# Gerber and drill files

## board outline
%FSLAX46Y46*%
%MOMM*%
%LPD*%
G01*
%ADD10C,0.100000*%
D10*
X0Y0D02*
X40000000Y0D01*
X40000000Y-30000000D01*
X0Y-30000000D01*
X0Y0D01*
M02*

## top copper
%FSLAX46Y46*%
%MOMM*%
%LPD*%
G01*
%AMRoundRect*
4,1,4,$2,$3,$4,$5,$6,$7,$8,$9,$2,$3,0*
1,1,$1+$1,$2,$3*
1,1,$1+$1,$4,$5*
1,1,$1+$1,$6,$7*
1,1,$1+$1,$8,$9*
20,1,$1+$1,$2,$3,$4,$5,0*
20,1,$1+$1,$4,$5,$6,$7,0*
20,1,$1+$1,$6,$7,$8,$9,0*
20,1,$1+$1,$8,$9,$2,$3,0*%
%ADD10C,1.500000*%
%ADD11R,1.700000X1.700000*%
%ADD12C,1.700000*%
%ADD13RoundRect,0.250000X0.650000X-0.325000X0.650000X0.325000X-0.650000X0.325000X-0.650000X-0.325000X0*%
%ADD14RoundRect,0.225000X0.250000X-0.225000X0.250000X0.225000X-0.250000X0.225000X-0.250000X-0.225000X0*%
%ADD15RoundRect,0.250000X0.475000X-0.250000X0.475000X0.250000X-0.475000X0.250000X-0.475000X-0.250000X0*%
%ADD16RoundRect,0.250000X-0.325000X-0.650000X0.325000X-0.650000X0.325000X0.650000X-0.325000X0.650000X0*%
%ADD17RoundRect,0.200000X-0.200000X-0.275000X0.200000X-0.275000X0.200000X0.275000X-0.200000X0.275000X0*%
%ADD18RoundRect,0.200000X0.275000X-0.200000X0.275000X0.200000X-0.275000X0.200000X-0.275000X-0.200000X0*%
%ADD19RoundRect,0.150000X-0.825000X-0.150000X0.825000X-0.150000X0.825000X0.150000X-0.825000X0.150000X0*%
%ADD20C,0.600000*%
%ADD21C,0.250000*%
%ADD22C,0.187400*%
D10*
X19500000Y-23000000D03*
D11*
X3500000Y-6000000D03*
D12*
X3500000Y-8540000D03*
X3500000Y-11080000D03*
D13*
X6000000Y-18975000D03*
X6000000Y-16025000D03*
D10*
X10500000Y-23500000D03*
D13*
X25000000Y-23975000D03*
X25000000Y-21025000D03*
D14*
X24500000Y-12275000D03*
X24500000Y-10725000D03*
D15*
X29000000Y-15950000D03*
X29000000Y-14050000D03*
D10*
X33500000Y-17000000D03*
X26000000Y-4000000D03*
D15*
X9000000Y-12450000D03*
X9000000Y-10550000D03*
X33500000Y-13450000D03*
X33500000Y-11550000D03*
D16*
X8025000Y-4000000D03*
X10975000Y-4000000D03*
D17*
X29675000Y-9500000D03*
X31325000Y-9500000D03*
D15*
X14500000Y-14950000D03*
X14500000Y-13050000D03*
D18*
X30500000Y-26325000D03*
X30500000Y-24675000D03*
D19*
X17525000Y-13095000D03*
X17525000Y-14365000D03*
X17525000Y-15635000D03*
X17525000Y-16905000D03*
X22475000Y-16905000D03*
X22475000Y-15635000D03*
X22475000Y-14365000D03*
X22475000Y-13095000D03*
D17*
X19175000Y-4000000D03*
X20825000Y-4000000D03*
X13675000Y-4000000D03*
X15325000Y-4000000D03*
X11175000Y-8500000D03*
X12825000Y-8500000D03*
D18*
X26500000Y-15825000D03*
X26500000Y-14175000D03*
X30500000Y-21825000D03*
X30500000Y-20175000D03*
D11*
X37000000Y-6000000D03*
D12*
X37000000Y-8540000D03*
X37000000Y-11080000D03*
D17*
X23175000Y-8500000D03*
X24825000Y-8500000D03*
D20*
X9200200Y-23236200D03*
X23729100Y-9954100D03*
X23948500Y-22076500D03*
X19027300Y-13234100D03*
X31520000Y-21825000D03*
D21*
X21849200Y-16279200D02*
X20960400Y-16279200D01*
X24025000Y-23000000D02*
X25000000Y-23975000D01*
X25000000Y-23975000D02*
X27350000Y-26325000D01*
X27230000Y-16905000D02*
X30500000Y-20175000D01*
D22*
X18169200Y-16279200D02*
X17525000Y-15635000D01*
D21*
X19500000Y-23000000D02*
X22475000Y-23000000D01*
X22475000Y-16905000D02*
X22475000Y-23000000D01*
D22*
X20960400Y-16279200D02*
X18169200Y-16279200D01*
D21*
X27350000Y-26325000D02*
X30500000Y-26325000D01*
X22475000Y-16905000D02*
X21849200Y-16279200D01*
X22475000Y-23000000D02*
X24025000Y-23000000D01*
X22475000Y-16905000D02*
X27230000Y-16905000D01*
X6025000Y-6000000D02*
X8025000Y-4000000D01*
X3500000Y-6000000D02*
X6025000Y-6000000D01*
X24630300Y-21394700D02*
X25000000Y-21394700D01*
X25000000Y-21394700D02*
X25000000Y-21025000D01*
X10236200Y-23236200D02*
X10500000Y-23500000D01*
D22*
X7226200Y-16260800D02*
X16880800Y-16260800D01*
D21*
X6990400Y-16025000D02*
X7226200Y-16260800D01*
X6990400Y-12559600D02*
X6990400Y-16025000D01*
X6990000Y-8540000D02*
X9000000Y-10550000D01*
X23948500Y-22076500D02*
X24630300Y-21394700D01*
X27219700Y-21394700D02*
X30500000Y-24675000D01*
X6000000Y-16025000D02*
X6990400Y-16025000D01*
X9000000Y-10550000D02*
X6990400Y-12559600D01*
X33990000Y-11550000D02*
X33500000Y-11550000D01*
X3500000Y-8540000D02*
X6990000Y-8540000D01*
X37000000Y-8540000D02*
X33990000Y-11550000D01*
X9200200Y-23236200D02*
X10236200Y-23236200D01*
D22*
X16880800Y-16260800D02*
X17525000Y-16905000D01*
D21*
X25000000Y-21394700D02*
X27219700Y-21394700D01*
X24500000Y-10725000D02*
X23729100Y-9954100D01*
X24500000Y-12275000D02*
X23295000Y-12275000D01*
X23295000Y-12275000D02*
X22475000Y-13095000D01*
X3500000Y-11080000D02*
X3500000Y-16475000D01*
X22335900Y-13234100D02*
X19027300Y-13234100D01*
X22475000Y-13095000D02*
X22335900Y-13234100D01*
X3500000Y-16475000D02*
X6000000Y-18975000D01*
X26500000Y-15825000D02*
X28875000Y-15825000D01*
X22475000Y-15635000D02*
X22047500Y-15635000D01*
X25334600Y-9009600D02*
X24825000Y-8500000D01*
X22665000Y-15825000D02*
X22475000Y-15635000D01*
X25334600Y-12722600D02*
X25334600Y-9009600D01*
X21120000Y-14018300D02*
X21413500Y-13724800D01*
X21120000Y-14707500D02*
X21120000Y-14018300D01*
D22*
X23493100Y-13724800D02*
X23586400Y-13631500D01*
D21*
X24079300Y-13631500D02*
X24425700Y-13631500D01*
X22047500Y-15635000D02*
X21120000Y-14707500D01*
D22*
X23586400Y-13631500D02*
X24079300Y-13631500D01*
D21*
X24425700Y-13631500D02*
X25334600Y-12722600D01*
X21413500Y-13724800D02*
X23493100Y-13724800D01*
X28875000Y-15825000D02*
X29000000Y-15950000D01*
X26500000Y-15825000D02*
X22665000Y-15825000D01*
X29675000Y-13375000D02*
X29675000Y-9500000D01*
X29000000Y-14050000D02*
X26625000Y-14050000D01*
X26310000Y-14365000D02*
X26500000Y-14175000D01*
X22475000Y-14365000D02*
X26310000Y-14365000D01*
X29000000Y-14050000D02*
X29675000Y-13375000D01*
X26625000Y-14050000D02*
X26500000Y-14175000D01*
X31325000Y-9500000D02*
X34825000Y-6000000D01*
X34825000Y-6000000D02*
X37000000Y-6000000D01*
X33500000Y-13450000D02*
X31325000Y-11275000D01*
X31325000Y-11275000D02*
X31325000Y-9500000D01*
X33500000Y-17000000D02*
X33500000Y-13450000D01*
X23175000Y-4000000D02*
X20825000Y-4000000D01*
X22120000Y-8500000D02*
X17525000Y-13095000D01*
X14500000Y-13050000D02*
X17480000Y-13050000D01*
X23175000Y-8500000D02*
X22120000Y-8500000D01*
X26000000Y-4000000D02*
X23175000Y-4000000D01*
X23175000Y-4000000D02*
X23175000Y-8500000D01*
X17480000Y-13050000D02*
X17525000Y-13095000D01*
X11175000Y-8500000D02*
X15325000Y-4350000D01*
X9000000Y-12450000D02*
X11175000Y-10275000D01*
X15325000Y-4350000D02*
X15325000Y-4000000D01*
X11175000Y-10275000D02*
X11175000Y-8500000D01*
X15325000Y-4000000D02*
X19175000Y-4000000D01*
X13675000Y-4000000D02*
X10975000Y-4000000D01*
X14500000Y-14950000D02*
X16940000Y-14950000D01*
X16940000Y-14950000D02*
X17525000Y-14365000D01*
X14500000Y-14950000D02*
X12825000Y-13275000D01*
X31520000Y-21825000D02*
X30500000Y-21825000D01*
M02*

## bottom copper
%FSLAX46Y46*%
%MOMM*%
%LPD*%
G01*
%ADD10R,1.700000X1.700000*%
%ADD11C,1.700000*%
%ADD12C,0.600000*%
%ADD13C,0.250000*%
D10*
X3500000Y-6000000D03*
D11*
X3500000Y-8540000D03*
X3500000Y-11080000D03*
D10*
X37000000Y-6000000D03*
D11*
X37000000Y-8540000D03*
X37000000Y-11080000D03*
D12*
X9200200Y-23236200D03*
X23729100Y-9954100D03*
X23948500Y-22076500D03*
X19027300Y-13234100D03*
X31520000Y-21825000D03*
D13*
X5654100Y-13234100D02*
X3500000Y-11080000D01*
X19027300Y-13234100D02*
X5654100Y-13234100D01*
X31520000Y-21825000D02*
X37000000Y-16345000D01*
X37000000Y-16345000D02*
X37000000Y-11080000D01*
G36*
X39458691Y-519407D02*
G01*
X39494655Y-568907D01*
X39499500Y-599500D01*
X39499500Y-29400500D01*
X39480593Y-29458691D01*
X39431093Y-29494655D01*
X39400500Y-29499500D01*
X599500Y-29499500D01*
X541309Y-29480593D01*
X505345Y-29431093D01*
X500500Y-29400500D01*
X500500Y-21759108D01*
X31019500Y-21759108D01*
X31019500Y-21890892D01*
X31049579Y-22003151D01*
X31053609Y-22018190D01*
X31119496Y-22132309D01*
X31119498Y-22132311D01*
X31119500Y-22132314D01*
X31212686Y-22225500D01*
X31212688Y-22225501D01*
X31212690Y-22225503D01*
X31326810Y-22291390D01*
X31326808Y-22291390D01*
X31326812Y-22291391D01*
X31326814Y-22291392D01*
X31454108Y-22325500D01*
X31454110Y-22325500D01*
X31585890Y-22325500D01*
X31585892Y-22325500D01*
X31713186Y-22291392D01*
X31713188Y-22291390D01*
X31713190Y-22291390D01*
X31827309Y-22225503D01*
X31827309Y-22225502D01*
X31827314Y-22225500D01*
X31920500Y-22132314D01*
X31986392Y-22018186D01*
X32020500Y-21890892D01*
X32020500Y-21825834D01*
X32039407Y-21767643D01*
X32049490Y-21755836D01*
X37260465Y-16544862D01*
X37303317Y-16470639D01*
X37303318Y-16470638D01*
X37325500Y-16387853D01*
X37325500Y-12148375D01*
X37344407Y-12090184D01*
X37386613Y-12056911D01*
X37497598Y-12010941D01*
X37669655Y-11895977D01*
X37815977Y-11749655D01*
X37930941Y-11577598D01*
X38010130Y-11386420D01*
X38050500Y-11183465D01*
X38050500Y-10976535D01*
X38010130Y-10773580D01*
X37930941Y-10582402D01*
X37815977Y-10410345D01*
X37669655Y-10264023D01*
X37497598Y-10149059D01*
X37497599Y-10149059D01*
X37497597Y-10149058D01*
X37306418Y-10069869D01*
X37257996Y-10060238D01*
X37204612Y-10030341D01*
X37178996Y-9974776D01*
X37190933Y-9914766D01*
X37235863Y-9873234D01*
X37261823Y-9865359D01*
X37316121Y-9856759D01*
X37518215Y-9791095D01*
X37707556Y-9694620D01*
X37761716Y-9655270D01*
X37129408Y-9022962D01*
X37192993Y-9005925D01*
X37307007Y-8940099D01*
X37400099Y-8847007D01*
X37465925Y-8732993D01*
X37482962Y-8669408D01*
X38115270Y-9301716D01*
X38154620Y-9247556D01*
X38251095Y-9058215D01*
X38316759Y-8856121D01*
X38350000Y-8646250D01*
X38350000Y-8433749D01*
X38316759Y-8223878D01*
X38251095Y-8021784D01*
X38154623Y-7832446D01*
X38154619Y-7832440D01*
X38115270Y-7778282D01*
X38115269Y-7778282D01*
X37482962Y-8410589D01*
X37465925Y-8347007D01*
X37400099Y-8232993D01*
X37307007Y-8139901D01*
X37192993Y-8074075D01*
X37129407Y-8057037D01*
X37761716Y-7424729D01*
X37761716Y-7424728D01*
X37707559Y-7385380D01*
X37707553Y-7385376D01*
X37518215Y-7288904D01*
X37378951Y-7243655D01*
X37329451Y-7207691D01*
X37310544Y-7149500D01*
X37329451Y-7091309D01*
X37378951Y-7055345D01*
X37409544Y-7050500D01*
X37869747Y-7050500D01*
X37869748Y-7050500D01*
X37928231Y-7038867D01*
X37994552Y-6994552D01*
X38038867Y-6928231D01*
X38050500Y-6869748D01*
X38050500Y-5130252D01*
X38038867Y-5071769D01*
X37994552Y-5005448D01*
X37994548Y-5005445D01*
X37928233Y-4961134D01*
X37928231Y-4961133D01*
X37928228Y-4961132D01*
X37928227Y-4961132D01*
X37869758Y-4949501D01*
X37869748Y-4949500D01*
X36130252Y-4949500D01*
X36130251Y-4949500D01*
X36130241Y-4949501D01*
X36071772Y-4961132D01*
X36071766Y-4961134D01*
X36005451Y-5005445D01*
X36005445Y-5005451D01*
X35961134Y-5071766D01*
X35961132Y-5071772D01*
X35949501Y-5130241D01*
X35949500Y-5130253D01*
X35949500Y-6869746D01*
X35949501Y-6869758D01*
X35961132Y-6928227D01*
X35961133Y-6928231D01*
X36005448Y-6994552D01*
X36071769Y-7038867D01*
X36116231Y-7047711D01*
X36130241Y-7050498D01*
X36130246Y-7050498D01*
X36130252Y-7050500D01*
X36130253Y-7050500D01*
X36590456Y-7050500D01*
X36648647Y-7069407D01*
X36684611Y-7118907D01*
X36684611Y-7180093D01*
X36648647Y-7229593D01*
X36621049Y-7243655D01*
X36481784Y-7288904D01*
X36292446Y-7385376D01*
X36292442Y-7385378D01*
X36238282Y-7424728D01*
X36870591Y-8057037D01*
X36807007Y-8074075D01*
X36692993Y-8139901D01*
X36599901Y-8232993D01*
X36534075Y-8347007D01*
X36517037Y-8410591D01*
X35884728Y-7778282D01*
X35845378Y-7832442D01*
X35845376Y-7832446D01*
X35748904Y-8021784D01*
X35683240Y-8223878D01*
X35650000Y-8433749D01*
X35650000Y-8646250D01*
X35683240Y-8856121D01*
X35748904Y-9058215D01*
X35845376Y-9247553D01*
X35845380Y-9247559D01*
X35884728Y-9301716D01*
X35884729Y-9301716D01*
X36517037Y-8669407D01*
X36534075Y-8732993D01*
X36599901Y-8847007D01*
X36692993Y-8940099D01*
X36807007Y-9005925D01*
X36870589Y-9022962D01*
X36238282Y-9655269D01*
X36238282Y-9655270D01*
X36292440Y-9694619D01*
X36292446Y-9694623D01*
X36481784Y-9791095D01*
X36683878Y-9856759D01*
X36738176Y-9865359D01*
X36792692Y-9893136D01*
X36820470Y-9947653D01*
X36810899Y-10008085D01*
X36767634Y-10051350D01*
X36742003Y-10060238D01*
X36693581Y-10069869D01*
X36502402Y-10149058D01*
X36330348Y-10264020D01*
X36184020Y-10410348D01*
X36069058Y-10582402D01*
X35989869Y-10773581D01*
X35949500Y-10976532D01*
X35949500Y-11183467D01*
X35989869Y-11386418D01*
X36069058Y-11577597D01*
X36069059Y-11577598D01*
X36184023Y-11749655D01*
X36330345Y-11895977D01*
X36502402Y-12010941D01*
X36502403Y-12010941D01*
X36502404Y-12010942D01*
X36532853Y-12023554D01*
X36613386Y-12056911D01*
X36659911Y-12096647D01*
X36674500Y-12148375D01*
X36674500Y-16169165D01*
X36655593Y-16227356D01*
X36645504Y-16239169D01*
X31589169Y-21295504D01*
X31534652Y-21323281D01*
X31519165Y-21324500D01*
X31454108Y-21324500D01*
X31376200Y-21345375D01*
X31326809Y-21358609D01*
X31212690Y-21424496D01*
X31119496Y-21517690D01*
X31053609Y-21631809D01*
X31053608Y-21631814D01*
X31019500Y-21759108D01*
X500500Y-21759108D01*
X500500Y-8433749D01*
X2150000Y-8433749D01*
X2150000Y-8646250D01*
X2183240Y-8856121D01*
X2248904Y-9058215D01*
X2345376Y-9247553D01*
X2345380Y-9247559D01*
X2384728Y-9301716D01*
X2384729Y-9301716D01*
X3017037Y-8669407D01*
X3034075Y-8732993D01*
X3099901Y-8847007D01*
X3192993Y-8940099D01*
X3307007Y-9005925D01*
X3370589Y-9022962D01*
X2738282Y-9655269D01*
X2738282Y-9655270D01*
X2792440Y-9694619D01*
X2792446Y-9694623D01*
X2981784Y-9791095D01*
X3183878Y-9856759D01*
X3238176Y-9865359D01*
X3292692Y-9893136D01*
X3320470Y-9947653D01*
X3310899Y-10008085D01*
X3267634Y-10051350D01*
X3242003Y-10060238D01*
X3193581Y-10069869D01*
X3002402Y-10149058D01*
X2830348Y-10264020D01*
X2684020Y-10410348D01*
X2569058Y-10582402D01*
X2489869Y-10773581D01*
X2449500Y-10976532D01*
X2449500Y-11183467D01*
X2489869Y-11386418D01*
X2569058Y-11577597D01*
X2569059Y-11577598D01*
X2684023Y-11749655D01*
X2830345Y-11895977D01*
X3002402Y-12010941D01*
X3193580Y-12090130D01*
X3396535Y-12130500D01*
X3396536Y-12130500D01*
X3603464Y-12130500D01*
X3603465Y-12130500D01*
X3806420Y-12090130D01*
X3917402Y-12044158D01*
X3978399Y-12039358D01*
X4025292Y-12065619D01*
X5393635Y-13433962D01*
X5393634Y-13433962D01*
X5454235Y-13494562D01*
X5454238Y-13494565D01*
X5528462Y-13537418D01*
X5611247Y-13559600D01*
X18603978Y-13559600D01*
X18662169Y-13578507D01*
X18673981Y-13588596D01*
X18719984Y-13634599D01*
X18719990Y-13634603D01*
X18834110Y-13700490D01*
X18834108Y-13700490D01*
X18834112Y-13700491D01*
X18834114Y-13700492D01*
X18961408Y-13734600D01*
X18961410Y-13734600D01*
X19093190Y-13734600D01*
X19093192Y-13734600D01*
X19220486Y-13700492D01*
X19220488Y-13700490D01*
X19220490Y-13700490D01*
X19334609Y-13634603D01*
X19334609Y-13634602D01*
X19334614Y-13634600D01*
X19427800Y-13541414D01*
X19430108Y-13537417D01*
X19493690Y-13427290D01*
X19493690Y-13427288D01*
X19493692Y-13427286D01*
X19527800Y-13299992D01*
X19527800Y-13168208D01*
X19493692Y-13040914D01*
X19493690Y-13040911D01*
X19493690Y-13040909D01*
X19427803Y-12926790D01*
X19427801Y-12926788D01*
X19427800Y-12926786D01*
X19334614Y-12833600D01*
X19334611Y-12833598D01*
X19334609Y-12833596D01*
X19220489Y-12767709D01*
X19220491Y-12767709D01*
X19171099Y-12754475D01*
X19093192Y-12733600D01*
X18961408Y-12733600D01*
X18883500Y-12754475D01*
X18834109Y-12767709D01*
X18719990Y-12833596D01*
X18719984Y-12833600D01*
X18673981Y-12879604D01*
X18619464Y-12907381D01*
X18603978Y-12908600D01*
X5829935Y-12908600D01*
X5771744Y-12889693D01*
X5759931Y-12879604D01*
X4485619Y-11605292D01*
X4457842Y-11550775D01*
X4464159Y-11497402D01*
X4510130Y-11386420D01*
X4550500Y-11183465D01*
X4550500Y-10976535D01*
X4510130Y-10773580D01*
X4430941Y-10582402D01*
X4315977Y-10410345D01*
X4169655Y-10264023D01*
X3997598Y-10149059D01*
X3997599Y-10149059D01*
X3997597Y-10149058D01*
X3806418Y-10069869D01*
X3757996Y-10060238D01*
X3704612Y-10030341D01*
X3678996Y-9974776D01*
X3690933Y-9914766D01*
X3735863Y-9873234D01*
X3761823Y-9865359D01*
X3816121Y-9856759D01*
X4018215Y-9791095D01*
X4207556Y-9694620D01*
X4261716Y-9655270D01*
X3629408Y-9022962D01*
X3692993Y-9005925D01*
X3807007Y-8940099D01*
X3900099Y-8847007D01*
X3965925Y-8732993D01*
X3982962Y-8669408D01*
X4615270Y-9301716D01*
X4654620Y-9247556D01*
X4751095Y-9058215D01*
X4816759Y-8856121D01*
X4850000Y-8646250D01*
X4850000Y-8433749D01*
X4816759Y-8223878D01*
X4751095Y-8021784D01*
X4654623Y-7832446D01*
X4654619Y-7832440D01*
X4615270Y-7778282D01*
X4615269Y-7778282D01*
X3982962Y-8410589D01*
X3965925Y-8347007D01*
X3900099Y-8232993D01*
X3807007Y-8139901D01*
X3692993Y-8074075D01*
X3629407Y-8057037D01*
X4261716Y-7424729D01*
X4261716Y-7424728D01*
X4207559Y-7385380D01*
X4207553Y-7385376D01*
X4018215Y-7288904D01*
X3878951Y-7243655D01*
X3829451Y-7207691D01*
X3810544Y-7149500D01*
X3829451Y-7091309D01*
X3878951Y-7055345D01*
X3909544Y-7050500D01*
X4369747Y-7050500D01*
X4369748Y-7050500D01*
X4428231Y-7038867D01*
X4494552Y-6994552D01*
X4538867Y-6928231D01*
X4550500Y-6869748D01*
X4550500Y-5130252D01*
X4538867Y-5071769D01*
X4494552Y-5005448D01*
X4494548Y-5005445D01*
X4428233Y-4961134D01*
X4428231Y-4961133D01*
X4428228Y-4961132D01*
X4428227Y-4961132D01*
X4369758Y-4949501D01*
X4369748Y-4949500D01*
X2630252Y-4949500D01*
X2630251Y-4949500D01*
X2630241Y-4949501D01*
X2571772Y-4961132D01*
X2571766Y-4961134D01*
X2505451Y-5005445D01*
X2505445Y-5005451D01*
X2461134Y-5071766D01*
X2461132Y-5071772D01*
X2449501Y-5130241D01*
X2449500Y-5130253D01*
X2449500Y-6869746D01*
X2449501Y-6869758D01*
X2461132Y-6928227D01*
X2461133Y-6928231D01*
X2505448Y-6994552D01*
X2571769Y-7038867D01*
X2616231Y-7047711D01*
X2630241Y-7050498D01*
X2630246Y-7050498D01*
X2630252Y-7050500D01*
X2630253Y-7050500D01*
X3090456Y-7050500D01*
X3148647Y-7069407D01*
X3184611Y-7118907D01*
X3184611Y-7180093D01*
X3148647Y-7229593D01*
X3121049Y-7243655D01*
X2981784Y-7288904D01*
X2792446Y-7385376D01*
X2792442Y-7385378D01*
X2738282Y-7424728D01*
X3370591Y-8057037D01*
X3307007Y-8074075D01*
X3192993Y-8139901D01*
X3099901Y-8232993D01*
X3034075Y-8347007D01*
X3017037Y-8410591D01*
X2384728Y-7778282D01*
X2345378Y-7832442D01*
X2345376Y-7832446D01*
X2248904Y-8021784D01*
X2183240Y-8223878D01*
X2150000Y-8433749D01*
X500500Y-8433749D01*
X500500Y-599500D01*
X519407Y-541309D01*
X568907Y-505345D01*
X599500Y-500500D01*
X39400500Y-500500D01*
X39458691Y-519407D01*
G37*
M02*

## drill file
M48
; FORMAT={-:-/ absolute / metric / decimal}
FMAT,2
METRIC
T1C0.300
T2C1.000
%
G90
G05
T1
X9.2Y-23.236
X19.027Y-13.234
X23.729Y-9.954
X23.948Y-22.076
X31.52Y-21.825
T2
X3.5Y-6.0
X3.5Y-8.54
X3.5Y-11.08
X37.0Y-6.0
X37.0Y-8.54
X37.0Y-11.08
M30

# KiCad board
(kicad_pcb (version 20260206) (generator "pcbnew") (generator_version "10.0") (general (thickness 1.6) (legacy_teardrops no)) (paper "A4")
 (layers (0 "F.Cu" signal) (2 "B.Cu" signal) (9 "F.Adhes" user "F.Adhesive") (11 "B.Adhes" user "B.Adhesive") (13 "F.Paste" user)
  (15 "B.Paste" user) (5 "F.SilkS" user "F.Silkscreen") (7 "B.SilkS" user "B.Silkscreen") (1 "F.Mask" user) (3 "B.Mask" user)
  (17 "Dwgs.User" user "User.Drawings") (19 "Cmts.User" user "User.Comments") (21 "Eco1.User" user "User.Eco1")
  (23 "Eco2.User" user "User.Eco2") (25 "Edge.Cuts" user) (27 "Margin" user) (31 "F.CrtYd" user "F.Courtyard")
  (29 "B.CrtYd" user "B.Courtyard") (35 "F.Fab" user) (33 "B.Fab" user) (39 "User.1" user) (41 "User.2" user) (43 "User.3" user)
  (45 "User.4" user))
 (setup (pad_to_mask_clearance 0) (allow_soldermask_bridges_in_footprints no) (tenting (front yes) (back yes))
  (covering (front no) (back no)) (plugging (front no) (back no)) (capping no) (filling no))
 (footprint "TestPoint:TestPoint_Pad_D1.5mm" (layer "F.Cu") (at 19.5 23)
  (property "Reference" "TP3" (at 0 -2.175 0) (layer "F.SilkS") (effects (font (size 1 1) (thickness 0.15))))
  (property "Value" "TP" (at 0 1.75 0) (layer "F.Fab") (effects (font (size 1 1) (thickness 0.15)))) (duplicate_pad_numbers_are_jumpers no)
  (pad "1" smd circle (at 0 0) (size 1.5 1.5) (layers "F.Cu" "F.Mask") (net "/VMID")))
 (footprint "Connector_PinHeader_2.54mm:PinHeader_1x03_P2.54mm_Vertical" (layer "F.Cu") (at 3.5 6)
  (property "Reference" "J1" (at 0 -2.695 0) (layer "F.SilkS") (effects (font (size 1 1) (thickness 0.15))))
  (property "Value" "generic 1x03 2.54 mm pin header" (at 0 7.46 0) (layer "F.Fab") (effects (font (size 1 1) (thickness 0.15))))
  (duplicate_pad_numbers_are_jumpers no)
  (pad "1" thru_hole rect (at 0 0) (size 1.7 1.7) (drill 1) (layers "*.Cu" "*.Mask") (remove_unused_layers no) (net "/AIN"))
  (pad "2" thru_hole circle (at 0 2.54) (size 1.7 1.7) (drill 1) (layers "*.Cu" "*.Mask") (remove_unused_layers no) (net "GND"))
  (pad "3" thru_hole circle (at 0 5.08) (size 1.7 1.7) (drill 1) (layers "*.Cu" "*.Mask") (remove_unused_layers no) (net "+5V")))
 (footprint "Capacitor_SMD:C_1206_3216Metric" (layer "F.Cu") (at 6 17.5 90)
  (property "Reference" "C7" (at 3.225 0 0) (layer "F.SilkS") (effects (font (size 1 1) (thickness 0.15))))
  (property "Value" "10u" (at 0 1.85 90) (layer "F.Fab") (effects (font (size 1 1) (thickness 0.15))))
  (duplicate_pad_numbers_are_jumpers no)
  (pad "1" smd roundrect (at -1.475 0 90) (size 1.15 1.8) (layers "F.Cu" "F.Mask" "F.Paste") (roundrect_rratio 0.217391) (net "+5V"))
  (pad "2" smd roundrect (at 1.475 0 90) (size 1.15 1.8) (layers "F.Cu" "F.Mask" "F.Paste") (roundrect_rratio 0.217391) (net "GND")))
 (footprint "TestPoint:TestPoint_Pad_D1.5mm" (layer "F.Cu") (at 10.5 23.5)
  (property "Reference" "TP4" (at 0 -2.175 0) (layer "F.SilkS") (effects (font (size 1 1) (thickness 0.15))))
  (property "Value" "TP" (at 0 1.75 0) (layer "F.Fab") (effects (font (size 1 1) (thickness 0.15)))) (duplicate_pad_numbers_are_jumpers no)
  (pad "1" smd circle (at 0 0) (size 1.5 1.5) (layers "F.Cu" "F.Mask") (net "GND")))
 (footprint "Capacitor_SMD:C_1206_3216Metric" (layer "F.Cu") (at 25 22.5 90)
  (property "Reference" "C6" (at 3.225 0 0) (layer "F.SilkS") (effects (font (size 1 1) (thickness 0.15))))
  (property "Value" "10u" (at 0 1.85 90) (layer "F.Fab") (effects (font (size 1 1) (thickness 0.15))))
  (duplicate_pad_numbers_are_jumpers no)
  (pad "1" smd roundrect (at -1.475 0 90) (size 1.15 1.8) (layers "F.Cu" "F.Mask" "F.Paste") (roundrect_rratio 0.217391) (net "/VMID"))
  (pad "2" smd roundrect (at 1.475 0 90) (size 1.15 1.8) (layers "F.Cu" "F.Mask" "F.Paste") (roundrect_rratio 0.217391) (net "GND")))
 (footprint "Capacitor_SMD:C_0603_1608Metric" (layer "F.Cu") (at 24.5 11.5 90)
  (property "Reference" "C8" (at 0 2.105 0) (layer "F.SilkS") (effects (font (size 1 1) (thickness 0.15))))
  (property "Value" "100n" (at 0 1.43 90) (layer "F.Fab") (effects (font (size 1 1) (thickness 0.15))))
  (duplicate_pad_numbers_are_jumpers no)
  (pad "1" smd roundrect (at -0.775 0 90) (size 0.9 0.95) (layers "F.Cu" "F.Mask" "F.Paste") (roundrect_rratio 0.25) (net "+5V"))
  (pad "2" smd roundrect (at 0.775 0 90) (size 0.9 0.95) (layers "F.Cu" "F.Mask" "F.Paste") (roundrect_rratio 0.25) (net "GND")))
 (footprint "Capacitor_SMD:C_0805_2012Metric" (layer "F.Cu") (at 29 15 90)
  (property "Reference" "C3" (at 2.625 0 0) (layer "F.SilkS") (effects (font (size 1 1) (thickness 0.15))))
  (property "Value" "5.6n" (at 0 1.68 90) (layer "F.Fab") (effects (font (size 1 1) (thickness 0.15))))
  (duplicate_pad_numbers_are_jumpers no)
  (pad "1" smd roundrect (at -0.95 0 90) (size 1 1.45) (layers "F.Cu" "F.Mask" "F.Paste") (roundrect_rratio 0.25) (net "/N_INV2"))
  (pad "2" smd roundrect (at 0.95 0 90) (size 1 1.45) (layers "F.Cu" "F.Mask" "F.Paste") (roundrect_rratio 0.25) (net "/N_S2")))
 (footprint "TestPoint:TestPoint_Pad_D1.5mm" (layer "F.Cu") (at 33.5 17)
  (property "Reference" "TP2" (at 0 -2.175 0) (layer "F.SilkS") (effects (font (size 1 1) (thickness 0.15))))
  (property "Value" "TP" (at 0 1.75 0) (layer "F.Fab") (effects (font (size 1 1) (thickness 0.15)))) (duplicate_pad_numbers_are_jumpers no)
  (pad "1" smd circle (at 0 0) (size 1.5 1.5) (layers "F.Cu" "F.Mask") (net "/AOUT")))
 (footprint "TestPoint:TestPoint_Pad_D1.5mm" (layer "F.Cu") (at 26 4)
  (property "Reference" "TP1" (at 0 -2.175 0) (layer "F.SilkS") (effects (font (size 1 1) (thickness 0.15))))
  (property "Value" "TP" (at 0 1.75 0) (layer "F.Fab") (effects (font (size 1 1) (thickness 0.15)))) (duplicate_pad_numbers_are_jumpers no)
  (pad "1" smd circle (at 0 0) (size 1.5 1.5) (layers "F.Cu" "F.Mask") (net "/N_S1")))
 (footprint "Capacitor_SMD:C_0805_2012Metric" (layer "F.Cu") (at 9 11.5 90)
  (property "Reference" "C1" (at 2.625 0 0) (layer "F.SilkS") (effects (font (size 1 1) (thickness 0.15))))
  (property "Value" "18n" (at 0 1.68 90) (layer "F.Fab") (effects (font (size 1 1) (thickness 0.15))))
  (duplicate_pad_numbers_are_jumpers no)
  (pad "1" smd roundrect (at -0.95 0 90) (size 1 1.45) (layers "F.Cu" "F.Mask" "F.Paste") (roundrect_rratio 0.25) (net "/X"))
  (pad "2" smd roundrect (at 0.95 0 90) (size 1 1.45) (layers "F.Cu" "F.Mask" "F.Paste") (roundrect_rratio 0.25) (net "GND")))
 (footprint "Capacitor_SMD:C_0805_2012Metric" (layer "F.Cu") (at 33.5 12.5 90)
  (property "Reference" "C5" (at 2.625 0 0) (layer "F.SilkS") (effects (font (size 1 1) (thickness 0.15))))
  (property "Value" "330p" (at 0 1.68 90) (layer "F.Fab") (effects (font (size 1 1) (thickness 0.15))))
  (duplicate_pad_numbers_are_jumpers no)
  (pad "1" smd roundrect (at -0.95 0 90) (size 1 1.45) (layers "F.Cu" "F.Mask" "F.Paste") (roundrect_rratio 0.25) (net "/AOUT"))
  (pad "2" smd roundrect (at 0.95 0 90) (size 1 1.45) (layers "F.Cu" "F.Mask" "F.Paste") (roundrect_rratio 0.25) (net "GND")))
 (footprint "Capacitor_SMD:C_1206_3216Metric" (layer "F.Cu") (at 9.5 4)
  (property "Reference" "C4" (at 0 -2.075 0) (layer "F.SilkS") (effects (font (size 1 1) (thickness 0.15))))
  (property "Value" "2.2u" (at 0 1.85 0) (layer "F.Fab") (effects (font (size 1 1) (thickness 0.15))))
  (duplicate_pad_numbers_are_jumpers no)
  (pad "1" smd roundrect (at -1.475 0) (size 1.15 1.8) (layers "F.Cu" "F.Mask" "F.Paste") (roundrect_rratio 0.217391) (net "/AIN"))
  (pad "2" smd roundrect (at 1.475 0) (size 1.15 1.8) (layers "F.Cu" "F.Mask" "F.Paste") (roundrect_rratio 0.217391) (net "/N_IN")))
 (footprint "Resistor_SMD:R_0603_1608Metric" (layer "F.Cu") (at 30.5 9.5)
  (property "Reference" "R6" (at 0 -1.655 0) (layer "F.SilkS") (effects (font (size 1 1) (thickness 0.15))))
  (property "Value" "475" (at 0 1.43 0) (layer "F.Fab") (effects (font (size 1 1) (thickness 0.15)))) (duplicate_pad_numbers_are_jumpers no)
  (pad "1" smd roundrect (at -0.825 0) (size 0.8 0.95) (layers "F.Cu" "F.Mask" "F.Paste") (roundrect_rratio 0.25) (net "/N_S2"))
  (pad "2" smd roundrect (at 0.825 0) (size 0.8 0.95) (layers "F.Cu" "F.Mask" "F.Paste") (roundrect_rratio 0.25) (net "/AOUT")))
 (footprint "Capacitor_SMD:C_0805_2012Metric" (layer "F.Cu") (at 14.5 14 90)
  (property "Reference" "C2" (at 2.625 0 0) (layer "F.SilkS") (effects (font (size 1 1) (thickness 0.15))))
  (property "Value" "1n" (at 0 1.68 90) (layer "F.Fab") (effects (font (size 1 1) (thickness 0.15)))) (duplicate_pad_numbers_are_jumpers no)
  (pad "1" smd roundrect (at -0.95 0 90) (size 1 1.45) (layers "F.Cu" "F.Mask" "F.Paste") (roundrect_rratio 0.25) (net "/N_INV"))
  (pad "2" smd roundrect (at 0.95 0 90) (size 1 1.45) (layers "F.Cu" "F.Mask" "F.Paste") (roundrect_rratio 0.25) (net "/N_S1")))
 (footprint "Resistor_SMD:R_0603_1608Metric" (layer "F.Cu") (at 30.5 25.5 90)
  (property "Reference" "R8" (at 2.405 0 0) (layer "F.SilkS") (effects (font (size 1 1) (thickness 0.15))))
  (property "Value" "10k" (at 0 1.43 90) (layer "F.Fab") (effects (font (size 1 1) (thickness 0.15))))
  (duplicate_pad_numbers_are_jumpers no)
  (pad "1" smd roundrect (at -0.825 0 90) (size 0.8 0.95) (layers "F.Cu" "F.Mask" "F.Paste") (roundrect_rratio 0.25) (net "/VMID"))
  (pad "2" smd roundrect (at 0.825 0 90) (size 0.8 0.95) (layers "F.Cu" "F.Mask" "F.Paste") (roundrect_rratio 0.25) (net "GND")))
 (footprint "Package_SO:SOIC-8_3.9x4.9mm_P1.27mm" (layer "F.Cu") (at 20 15)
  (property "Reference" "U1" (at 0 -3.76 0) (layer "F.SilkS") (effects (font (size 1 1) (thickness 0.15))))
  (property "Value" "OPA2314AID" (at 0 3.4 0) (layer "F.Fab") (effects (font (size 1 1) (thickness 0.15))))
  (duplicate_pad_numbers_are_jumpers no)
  (pad "1" smd roundrect (at -2.475 -1.905) (size 1.95 0.6) (layers "F.Cu" "F.Mask" "F.Paste") (roundrect_rratio 0.25) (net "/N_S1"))
  (pad "2" smd roundrect (at -2.475 -0.635) (size 1.95 0.6) (layers "F.Cu" "F.Mask" "F.Paste") (roundrect_rratio 0.25) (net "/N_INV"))
  (pad "3" smd roundrect (at -2.475 0.635) (size 1.95 0.6) (layers "F.Cu" "F.Mask" "F.Paste") (roundrect_rratio 0.25) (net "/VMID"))
  (pad "4" smd roundrect (at -2.475 1.905) (size 1.95 0.6) (layers "F.Cu" "F.Mask" "F.Paste") (roundrect_rratio 0.25) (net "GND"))
  (pad "5" smd roundrect (at 2.475 1.905) (size 1.95 0.6) (layers "F.Cu" "F.Mask" "F.Paste") (roundrect_rratio 0.25) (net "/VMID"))
  (pad "6" smd roundrect (at 2.475 0.635) (size 1.95 0.6) (layers "F.Cu" "F.Mask" "F.Paste") (roundrect_rratio 0.25) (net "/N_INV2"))
  (pad "7" smd roundrect (at 2.475 -0.635) (size 1.95 0.6) (layers "F.Cu" "F.Mask" "F.Paste") (roundrect_rratio 0.25) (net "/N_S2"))
  (pad "8" smd roundrect (at 2.475 -1.905) (size 1.95 0.6) (layers "F.Cu" "F.Mask" "F.Paste") (roundrect_rratio 0.25) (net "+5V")))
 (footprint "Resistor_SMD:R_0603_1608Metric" (layer "F.Cu") (at 20 4)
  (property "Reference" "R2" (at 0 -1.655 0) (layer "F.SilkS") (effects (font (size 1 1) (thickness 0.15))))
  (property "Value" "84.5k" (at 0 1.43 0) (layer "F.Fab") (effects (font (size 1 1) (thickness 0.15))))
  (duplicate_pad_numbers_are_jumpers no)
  (pad "1" smd roundrect (at -0.825 0) (size 0.8 0.95) (layers "F.Cu" "F.Mask" "F.Paste") (roundrect_rratio 0.25) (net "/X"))
  (pad "2" smd roundrect (at 0.825 0) (size 0.8 0.95) (layers "F.Cu" "F.Mask" "F.Paste") (roundrect_rratio 0.25) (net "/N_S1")))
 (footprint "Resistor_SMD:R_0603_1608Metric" (layer "F.Cu") (at 14.5 4)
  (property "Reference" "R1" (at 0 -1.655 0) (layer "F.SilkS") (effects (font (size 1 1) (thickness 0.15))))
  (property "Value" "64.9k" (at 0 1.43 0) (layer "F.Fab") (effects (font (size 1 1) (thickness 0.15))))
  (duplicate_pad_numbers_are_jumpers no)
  (pad "1" smd roundrect (at -0.825 0) (size 0.8 0.95) (layers "F.Cu" "F.Mask" "F.Paste") (roundrect_rratio 0.25) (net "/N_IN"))
  (pad "2" smd roundrect (at 0.825 0) (size 0.8 0.95) (layers "F.Cu" "F.Mask" "F.Paste") (roundrect_rratio 0.25) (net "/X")))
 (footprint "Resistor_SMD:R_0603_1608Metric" (layer "F.Cu") (at 12 8.5)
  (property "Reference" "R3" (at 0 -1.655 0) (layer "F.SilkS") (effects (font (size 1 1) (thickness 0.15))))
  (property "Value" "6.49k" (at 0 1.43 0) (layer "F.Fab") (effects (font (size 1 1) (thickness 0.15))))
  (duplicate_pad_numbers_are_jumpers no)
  (pad "1" smd roundrect (at -0.825 0) (size 0.8 0.95) (layers "F.Cu" "F.Mask" "F.Paste") (roundrect_rratio 0.25) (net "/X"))
  (pad "2" smd roundrect (at 0.825 0) (size 0.8 0.95) (layers "F.Cu" "F.Mask" "F.Paste") (roundrect_rratio 0.25) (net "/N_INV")))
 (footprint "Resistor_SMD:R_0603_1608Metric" (layer "F.Cu") (at 26.5 15 90)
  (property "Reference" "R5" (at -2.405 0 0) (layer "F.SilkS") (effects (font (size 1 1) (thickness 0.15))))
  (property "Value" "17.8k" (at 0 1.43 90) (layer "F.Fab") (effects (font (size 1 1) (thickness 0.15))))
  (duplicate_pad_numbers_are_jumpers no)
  (pad "1" smd roundrect (at -0.825 0 90) (size 0.8 0.95) (layers "F.Cu" "F.Mask" "F.Paste") (roundrect_rratio 0.25) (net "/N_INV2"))
  (pad "2" smd roundrect (at 0.825 0 90) (size 0.8 0.95) (layers "F.Cu" "F.Mask" "F.Paste") (roundrect_rratio 0.25) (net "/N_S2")))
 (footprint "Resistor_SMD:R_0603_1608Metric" (layer "F.Cu") (at 30.5 21 90)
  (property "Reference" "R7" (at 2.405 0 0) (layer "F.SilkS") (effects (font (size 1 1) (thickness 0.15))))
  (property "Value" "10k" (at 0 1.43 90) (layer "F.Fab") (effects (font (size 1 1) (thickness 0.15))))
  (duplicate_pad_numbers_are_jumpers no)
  (pad "1" smd roundrect (at -0.825 0 90) (size 0.8 0.95) (layers "F.Cu" "F.Mask" "F.Paste") (roundrect_rratio 0.25) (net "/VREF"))
  (pad "2" smd roundrect (at 0.825 0 90) (size 0.8 0.95) (layers "F.Cu" "F.Mask" "F.Paste") (roundrect_rratio 0.25) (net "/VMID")))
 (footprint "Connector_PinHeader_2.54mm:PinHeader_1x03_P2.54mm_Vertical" (layer "F.Cu") (at 37 6)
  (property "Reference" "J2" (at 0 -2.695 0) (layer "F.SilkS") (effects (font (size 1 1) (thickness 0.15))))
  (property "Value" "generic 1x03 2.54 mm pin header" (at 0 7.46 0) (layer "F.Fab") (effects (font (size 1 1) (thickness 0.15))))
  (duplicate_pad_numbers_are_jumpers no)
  (pad "1" thru_hole rect (at 0 0) (size 1.7 1.7) (drill 1) (layers "*.Cu" "*.Mask") (remove_unused_layers no) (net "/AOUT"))
  (pad "2" thru_hole circle (at 0 2.54) (size 1.7 1.7) (drill 1) (layers "*.Cu" "*.Mask") (remove_unused_layers no) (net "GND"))
  (pad "3" thru_hole circle (at 0 5.08) (size 1.7 1.7) (drill 1) (layers "*.Cu" "*.Mask") (remove_unused_layers no) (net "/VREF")))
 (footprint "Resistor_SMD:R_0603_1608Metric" (layer "F.Cu") (at 24 8.5)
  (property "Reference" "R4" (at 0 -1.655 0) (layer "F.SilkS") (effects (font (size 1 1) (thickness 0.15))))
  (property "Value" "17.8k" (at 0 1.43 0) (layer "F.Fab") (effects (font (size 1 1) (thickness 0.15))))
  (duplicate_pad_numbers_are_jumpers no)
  (pad "1" smd roundrect (at -0.825 0) (size 0.8 0.95) (layers "F.Cu" "F.Mask" "F.Paste") (roundrect_rratio 0.25) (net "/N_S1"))
  (pad "2" smd roundrect (at 0.825 0) (size 0.8 0.95) (layers "F.Cu" "F.Mask" "F.Paste") (roundrect_rratio 0.25) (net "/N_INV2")))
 (gr_rect (start 0 0) (end 40 30) (stroke (width 0.1) (type default)) (fill no) (layer "Edge.Cuts"))
 (segment (start 21.8492 16.2792) (end 20.9604 16.2792) (width 0.25) (layer "F.Cu") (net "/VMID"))
 (segment (start 24.025 23) (end 25 23.975) (width 0.25) (layer "F.Cu") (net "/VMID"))
 (segment (start 25 23.975) (end 27.35 26.325) (width 0.25) (layer "F.Cu") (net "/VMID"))
 (segment (start 27.23 16.905) (end 30.5 20.175) (width 0.25) (layer "F.Cu") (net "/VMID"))
 (segment (start 18.1692 16.2792) (end 17.525 15.635) (width 0.1874) (layer "F.Cu") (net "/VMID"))
 (segment (start 19.5 23) (end 22.475 23) (width 0.25) (layer "F.Cu") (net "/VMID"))
 (segment (start 22.475 16.905) (end 22.475 23) (width 0.25) (layer "F.Cu") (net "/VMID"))
 (segment (start 20.9604 16.2792) (end 18.1692 16.2792) (width 0.1874) (layer "F.Cu") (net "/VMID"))
 (segment (start 27.35 26.325) (end 30.5 26.325) (width 0.25) (layer "F.Cu") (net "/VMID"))
 (segment (start 22.475 16.905) (end 21.8492 16.2792) (width 0.25) (layer "F.Cu") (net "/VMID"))
 (segment (start 22.475 23) (end 24.025 23) (width 0.25) (layer "F.Cu") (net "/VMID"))
 (segment (start 22.475 16.905) (end 27.23 16.905) (width 0.25) (layer "F.Cu") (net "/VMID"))
 (segment (start 6.025 6) (end 8.025 4) (width 0.25) (layer "F.Cu") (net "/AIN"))
 (segment (start 3.5 6) (end 6.025 6) (width 0.25) (layer "F.Cu") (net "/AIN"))
 (segment (start 24.6303 21.3947) (end 25 21.3947) (width 0.25) (layer "F.Cu") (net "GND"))
 (segment (start 25 21.3947) (end 25 21.025) (width 0.25) (layer "F.Cu") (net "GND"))
 (segment (start 10.2362 23.2362) (end 10.5 23.5) (width 0.25) (layer "F.Cu") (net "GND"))
 (segment (start 7.2262 16.2608) (end 16.8808 16.2608) (width 0.1874) (layer "F.Cu") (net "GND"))
 (segment (start 6.9904 16.025) (end 7.2262 16.2608) (width 0.25) (layer "F.Cu") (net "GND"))
 (segment (start 6.9904 12.5596) (end 6.9904 16.025) (width 0.25) (layer "F.Cu") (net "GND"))
 (segment (start 6.99 8.54) (end 9 10.55) (width 0.25) (layer "F.Cu") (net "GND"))
 (segment (start 23.9485 22.0765) (end 24.6303 21.3947) (width 0.25) (layer "F.Cu") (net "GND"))
 (segment (start 27.2197 21.3947) (end 30.5 24.675) (width 0.25) (layer "F.Cu") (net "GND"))
 (segment (start 6 16.025) (end 6.9904 16.025) (width 0.25) (layer "F.Cu") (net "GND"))
 (segment (start 9 10.55) (end 6.9904 12.5596) (width 0.25) (layer "F.Cu") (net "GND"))
 (segment (start 33.99 11.55) (end 33.5 11.55) (width 0.25) (layer "F.Cu") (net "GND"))
 (segment (start 3.5 8.54) (end 6.99 8.54) (width 0.25) (layer "F.Cu") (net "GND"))
 (segment (start 37 8.54) (end 33.99 11.55) (width 0.25) (layer "F.Cu") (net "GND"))
 (segment (start 9.2002 23.2362) (end 10.2362 23.2362) (width 0.25) (layer "F.Cu") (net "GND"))
 (segment (start 16.8808 16.2608) (end 17.525 16.905) (width 0.1874) (layer "F.Cu") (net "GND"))
 (segment (start 25 21.3947) (end 27.2197 21.3947) (width 0.25) (layer "F.Cu") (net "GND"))
 (segment (start 24.5 10.725) (end 23.7291 9.9541) (width 0.25) (layer "F.Cu") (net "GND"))
 (via (at 9.2002 23.2362) (size 0.6) (drill 0.3) (layers "F.Cu" "B.Cu") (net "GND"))
 (via (at 23.7291 9.9541) (size 0.6) (drill 0.3) (layers "F.Cu" "B.Cu") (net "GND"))
 (via (at 23.9485 22.0765) (size 0.6) (drill 0.3) (layers "F.Cu" "B.Cu") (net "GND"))
 (segment (start 24.5 12.275) (end 23.295 12.275) (width 0.25) (layer "F.Cu") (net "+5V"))
 (segment (start 23.295 12.275) (end 22.475 13.095) (width 0.25) (layer "F.Cu") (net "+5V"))
 (segment (start 3.5 11.08) (end 3.5 16.475) (width 0.25) (layer "F.Cu") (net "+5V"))
 (segment (start 22.3359 13.2341) (end 19.0273 13.2341) (width 0.25) (layer "F.Cu") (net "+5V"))
 (segment (start 22.475 13.095) (end 22.3359 13.2341) (width 0.25) (layer "F.Cu") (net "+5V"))
 (segment (start 3.5 16.475) (end 6 18.975) (width 0.25) (layer "F.Cu") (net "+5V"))
 (via (at 19.0273 13.2341) (size 0.6) (drill 0.3) (layers "F.Cu" "B.Cu") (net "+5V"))
 (segment (start 5.6541 13.2341) (end 3.5 11.08) (width 0.25) (layer "B.Cu") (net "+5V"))
 (segment (start 19.0273 13.2341) (end 5.6541 13.2341) (width 0.25) (layer "B.Cu") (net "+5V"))
 (segment (start 26.5 15.825) (end 28.875 15.825) (width 0.25) (layer "F.Cu") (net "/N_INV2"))
 (segment (start 22.475 15.635) (end 22.0475 15.635) (width 0.25) (layer "F.Cu") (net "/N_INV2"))
 (segment (start 25.3346 9.0096) (end 24.825 8.5) (width 0.25) (layer "F.Cu") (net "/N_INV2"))
 (segment (start 22.665 15.825) (end 22.475 15.635) (width 0.25) (layer "F.Cu") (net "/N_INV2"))
 (segment (start 25.3346 12.7226) (end 25.3346 9.0096) (width 0.25) (layer "F.Cu") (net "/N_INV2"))
 (segment (start 21.12 14.0183) (end 21.4135 13.7248) (width 0.25) (layer "F.Cu") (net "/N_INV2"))
 (segment (start 21.12 14.7075) (end 21.12 14.0183) (width 0.25) (layer "F.Cu") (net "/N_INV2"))
 (segment (start 23.4931 13.7248) (end 23.5864 13.6315) (width 0.1874) (layer "F.Cu") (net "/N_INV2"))
 (segment (start 24.0793 13.6315) (end 24.4257 13.6315) (width 0.25) (layer "F.Cu") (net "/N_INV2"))
 (segment (start 22.0475 15.635) (end 21.12 14.7075) (width 0.25) (layer "F.Cu") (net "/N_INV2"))
 (segment (start 23.5864 13.6315) (end 24.0793 13.6315) (width 0.1874) (layer "F.Cu") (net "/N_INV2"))
 (segment (start 24.4257 13.6315) (end 25.3346 12.7226) (width 0.25) (layer "F.Cu") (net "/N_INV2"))
 (segment (start 21.4135 13.7248) (end 23.4931 13.7248) (width 0.25) (layer "F.Cu") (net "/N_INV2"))
 (segment (start 28.875 15.825) (end 29 15.95) (width 0.25) (layer "F.Cu") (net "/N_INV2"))
 (segment (start 26.5 15.825) (end 22.665 15.825) (width 0.25) (layer "F.Cu") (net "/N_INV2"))
 (segment (start 29.675 13.375) (end 29.675 9.5) (width 0.25) (layer "F.Cu") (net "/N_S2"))
 (segment (start 29 14.05) (end 26.625 14.05) (width 0.25) (layer "F.Cu") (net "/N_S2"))
 (segment (start 26.31 14.365) (end 26.5 14.175) (width 0.25) (layer "F.Cu") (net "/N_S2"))
 (segment (start 22.475 14.365) (end 26.31 14.365) (width 0.25) (layer "F.Cu") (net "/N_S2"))
 (segment (start 29 14.05) (end 29.675 13.375) (width 0.25) (layer "F.Cu") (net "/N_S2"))
 (segment (start 26.625 14.05) (end 26.5 14.175) (width 0.25) (layer "F.Cu") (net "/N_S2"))
 (segment (start 31.325 9.5) (end 34.825 6) (width 0.25) (layer "F.Cu") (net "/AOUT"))
 (segment (start 34.825 6) (end 37 6) (width 0.25) (layer "F.Cu") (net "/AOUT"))
 (segment (start 33.5 13.45) (end 31.325 11.275) (width 0.25) (layer "F.Cu") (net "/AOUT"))
 (segment (start 31.325 11.275) (end 31.325 9.5) (width 0.25) (layer "F.Cu") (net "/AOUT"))
 (segment (start 33.5 17) (end 33.5 13.45) (width 0.25) (layer "F.Cu") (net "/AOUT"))
 (segment (start 23.175 4) (end 20.825 4) (width 0.25) (layer "F.Cu") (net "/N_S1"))
 (segment (start 22.12 8.5) (end 17.525 13.095) (width 0.25) (layer "F.Cu") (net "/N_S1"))
 (segment (start 14.5 13.05) (end 17.48 13.05) (width 0.25) (layer "F.Cu") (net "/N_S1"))
 (segment (start 23.175 8.5) (end 22.12 8.5) (width 0.25) (layer "F.Cu") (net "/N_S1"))
 (segment (start 26 4) (end 23.175 4) (width 0.25) (layer "F.Cu") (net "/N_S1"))
 (segment (start 23.175 4) (end 23.175 8.5) (width 0.25) (layer "F.Cu") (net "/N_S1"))
 (segment (start 17.48 13.05) (end 17.525 13.095) (width 0.25) (layer "F.Cu") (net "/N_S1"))
 (segment (start 11.175 8.5) (end 15.325 4.35) (width 0.25) (layer "F.Cu") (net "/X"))
 (segment (start 9 12.45) (end 11.175 10.275) (width 0.25) (layer "F.Cu") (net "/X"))
 (segment (start 15.325 4.35) (end 15.325 4) (width 0.25) (layer "F.Cu") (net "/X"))
 (segment (start 11.175 10.275) (end 11.175 8.5) (width 0.25) (layer "F.Cu") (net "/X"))
 (segment (start 15.325 4) (end 19.175 4) (width 0.25) (layer "F.Cu") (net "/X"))
 (segment (start 13.675 4) (end 10.975 4) (width 0.25) (layer "F.Cu") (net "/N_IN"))
 (segment (start 14.5 14.95) (end 16.94 14.95) (width 0.25) (layer "F.Cu") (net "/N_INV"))
 (segment (start 16.94 14.95) (end 17.525 14.365) (width 0.25) (layer "F.Cu") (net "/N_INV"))
 (segment (start 14.5 14.95) (end 12.825 13.275) (width 0.25) (layer "F.Cu") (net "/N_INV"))
 (segment (start 31.52 21.825) (end 30.5 21.825) (width 0.25) (layer "F.Cu") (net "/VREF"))
 (via (at 31.52 21.825) (size 0.6) (drill 0.3) (layers "F.Cu" "B.Cu") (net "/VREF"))
 (segment (start 31.52 21.825) (end 37 16.345) (width 0.25) (layer "B.Cu") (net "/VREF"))
 (segment (start 37 16.345) (end 37 11.08) (width 0.25) (layer "B.Cu") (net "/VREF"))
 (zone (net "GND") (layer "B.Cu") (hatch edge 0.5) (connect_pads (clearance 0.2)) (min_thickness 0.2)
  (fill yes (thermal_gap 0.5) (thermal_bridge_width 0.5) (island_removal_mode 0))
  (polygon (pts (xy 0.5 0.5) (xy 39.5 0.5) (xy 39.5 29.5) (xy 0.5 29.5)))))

